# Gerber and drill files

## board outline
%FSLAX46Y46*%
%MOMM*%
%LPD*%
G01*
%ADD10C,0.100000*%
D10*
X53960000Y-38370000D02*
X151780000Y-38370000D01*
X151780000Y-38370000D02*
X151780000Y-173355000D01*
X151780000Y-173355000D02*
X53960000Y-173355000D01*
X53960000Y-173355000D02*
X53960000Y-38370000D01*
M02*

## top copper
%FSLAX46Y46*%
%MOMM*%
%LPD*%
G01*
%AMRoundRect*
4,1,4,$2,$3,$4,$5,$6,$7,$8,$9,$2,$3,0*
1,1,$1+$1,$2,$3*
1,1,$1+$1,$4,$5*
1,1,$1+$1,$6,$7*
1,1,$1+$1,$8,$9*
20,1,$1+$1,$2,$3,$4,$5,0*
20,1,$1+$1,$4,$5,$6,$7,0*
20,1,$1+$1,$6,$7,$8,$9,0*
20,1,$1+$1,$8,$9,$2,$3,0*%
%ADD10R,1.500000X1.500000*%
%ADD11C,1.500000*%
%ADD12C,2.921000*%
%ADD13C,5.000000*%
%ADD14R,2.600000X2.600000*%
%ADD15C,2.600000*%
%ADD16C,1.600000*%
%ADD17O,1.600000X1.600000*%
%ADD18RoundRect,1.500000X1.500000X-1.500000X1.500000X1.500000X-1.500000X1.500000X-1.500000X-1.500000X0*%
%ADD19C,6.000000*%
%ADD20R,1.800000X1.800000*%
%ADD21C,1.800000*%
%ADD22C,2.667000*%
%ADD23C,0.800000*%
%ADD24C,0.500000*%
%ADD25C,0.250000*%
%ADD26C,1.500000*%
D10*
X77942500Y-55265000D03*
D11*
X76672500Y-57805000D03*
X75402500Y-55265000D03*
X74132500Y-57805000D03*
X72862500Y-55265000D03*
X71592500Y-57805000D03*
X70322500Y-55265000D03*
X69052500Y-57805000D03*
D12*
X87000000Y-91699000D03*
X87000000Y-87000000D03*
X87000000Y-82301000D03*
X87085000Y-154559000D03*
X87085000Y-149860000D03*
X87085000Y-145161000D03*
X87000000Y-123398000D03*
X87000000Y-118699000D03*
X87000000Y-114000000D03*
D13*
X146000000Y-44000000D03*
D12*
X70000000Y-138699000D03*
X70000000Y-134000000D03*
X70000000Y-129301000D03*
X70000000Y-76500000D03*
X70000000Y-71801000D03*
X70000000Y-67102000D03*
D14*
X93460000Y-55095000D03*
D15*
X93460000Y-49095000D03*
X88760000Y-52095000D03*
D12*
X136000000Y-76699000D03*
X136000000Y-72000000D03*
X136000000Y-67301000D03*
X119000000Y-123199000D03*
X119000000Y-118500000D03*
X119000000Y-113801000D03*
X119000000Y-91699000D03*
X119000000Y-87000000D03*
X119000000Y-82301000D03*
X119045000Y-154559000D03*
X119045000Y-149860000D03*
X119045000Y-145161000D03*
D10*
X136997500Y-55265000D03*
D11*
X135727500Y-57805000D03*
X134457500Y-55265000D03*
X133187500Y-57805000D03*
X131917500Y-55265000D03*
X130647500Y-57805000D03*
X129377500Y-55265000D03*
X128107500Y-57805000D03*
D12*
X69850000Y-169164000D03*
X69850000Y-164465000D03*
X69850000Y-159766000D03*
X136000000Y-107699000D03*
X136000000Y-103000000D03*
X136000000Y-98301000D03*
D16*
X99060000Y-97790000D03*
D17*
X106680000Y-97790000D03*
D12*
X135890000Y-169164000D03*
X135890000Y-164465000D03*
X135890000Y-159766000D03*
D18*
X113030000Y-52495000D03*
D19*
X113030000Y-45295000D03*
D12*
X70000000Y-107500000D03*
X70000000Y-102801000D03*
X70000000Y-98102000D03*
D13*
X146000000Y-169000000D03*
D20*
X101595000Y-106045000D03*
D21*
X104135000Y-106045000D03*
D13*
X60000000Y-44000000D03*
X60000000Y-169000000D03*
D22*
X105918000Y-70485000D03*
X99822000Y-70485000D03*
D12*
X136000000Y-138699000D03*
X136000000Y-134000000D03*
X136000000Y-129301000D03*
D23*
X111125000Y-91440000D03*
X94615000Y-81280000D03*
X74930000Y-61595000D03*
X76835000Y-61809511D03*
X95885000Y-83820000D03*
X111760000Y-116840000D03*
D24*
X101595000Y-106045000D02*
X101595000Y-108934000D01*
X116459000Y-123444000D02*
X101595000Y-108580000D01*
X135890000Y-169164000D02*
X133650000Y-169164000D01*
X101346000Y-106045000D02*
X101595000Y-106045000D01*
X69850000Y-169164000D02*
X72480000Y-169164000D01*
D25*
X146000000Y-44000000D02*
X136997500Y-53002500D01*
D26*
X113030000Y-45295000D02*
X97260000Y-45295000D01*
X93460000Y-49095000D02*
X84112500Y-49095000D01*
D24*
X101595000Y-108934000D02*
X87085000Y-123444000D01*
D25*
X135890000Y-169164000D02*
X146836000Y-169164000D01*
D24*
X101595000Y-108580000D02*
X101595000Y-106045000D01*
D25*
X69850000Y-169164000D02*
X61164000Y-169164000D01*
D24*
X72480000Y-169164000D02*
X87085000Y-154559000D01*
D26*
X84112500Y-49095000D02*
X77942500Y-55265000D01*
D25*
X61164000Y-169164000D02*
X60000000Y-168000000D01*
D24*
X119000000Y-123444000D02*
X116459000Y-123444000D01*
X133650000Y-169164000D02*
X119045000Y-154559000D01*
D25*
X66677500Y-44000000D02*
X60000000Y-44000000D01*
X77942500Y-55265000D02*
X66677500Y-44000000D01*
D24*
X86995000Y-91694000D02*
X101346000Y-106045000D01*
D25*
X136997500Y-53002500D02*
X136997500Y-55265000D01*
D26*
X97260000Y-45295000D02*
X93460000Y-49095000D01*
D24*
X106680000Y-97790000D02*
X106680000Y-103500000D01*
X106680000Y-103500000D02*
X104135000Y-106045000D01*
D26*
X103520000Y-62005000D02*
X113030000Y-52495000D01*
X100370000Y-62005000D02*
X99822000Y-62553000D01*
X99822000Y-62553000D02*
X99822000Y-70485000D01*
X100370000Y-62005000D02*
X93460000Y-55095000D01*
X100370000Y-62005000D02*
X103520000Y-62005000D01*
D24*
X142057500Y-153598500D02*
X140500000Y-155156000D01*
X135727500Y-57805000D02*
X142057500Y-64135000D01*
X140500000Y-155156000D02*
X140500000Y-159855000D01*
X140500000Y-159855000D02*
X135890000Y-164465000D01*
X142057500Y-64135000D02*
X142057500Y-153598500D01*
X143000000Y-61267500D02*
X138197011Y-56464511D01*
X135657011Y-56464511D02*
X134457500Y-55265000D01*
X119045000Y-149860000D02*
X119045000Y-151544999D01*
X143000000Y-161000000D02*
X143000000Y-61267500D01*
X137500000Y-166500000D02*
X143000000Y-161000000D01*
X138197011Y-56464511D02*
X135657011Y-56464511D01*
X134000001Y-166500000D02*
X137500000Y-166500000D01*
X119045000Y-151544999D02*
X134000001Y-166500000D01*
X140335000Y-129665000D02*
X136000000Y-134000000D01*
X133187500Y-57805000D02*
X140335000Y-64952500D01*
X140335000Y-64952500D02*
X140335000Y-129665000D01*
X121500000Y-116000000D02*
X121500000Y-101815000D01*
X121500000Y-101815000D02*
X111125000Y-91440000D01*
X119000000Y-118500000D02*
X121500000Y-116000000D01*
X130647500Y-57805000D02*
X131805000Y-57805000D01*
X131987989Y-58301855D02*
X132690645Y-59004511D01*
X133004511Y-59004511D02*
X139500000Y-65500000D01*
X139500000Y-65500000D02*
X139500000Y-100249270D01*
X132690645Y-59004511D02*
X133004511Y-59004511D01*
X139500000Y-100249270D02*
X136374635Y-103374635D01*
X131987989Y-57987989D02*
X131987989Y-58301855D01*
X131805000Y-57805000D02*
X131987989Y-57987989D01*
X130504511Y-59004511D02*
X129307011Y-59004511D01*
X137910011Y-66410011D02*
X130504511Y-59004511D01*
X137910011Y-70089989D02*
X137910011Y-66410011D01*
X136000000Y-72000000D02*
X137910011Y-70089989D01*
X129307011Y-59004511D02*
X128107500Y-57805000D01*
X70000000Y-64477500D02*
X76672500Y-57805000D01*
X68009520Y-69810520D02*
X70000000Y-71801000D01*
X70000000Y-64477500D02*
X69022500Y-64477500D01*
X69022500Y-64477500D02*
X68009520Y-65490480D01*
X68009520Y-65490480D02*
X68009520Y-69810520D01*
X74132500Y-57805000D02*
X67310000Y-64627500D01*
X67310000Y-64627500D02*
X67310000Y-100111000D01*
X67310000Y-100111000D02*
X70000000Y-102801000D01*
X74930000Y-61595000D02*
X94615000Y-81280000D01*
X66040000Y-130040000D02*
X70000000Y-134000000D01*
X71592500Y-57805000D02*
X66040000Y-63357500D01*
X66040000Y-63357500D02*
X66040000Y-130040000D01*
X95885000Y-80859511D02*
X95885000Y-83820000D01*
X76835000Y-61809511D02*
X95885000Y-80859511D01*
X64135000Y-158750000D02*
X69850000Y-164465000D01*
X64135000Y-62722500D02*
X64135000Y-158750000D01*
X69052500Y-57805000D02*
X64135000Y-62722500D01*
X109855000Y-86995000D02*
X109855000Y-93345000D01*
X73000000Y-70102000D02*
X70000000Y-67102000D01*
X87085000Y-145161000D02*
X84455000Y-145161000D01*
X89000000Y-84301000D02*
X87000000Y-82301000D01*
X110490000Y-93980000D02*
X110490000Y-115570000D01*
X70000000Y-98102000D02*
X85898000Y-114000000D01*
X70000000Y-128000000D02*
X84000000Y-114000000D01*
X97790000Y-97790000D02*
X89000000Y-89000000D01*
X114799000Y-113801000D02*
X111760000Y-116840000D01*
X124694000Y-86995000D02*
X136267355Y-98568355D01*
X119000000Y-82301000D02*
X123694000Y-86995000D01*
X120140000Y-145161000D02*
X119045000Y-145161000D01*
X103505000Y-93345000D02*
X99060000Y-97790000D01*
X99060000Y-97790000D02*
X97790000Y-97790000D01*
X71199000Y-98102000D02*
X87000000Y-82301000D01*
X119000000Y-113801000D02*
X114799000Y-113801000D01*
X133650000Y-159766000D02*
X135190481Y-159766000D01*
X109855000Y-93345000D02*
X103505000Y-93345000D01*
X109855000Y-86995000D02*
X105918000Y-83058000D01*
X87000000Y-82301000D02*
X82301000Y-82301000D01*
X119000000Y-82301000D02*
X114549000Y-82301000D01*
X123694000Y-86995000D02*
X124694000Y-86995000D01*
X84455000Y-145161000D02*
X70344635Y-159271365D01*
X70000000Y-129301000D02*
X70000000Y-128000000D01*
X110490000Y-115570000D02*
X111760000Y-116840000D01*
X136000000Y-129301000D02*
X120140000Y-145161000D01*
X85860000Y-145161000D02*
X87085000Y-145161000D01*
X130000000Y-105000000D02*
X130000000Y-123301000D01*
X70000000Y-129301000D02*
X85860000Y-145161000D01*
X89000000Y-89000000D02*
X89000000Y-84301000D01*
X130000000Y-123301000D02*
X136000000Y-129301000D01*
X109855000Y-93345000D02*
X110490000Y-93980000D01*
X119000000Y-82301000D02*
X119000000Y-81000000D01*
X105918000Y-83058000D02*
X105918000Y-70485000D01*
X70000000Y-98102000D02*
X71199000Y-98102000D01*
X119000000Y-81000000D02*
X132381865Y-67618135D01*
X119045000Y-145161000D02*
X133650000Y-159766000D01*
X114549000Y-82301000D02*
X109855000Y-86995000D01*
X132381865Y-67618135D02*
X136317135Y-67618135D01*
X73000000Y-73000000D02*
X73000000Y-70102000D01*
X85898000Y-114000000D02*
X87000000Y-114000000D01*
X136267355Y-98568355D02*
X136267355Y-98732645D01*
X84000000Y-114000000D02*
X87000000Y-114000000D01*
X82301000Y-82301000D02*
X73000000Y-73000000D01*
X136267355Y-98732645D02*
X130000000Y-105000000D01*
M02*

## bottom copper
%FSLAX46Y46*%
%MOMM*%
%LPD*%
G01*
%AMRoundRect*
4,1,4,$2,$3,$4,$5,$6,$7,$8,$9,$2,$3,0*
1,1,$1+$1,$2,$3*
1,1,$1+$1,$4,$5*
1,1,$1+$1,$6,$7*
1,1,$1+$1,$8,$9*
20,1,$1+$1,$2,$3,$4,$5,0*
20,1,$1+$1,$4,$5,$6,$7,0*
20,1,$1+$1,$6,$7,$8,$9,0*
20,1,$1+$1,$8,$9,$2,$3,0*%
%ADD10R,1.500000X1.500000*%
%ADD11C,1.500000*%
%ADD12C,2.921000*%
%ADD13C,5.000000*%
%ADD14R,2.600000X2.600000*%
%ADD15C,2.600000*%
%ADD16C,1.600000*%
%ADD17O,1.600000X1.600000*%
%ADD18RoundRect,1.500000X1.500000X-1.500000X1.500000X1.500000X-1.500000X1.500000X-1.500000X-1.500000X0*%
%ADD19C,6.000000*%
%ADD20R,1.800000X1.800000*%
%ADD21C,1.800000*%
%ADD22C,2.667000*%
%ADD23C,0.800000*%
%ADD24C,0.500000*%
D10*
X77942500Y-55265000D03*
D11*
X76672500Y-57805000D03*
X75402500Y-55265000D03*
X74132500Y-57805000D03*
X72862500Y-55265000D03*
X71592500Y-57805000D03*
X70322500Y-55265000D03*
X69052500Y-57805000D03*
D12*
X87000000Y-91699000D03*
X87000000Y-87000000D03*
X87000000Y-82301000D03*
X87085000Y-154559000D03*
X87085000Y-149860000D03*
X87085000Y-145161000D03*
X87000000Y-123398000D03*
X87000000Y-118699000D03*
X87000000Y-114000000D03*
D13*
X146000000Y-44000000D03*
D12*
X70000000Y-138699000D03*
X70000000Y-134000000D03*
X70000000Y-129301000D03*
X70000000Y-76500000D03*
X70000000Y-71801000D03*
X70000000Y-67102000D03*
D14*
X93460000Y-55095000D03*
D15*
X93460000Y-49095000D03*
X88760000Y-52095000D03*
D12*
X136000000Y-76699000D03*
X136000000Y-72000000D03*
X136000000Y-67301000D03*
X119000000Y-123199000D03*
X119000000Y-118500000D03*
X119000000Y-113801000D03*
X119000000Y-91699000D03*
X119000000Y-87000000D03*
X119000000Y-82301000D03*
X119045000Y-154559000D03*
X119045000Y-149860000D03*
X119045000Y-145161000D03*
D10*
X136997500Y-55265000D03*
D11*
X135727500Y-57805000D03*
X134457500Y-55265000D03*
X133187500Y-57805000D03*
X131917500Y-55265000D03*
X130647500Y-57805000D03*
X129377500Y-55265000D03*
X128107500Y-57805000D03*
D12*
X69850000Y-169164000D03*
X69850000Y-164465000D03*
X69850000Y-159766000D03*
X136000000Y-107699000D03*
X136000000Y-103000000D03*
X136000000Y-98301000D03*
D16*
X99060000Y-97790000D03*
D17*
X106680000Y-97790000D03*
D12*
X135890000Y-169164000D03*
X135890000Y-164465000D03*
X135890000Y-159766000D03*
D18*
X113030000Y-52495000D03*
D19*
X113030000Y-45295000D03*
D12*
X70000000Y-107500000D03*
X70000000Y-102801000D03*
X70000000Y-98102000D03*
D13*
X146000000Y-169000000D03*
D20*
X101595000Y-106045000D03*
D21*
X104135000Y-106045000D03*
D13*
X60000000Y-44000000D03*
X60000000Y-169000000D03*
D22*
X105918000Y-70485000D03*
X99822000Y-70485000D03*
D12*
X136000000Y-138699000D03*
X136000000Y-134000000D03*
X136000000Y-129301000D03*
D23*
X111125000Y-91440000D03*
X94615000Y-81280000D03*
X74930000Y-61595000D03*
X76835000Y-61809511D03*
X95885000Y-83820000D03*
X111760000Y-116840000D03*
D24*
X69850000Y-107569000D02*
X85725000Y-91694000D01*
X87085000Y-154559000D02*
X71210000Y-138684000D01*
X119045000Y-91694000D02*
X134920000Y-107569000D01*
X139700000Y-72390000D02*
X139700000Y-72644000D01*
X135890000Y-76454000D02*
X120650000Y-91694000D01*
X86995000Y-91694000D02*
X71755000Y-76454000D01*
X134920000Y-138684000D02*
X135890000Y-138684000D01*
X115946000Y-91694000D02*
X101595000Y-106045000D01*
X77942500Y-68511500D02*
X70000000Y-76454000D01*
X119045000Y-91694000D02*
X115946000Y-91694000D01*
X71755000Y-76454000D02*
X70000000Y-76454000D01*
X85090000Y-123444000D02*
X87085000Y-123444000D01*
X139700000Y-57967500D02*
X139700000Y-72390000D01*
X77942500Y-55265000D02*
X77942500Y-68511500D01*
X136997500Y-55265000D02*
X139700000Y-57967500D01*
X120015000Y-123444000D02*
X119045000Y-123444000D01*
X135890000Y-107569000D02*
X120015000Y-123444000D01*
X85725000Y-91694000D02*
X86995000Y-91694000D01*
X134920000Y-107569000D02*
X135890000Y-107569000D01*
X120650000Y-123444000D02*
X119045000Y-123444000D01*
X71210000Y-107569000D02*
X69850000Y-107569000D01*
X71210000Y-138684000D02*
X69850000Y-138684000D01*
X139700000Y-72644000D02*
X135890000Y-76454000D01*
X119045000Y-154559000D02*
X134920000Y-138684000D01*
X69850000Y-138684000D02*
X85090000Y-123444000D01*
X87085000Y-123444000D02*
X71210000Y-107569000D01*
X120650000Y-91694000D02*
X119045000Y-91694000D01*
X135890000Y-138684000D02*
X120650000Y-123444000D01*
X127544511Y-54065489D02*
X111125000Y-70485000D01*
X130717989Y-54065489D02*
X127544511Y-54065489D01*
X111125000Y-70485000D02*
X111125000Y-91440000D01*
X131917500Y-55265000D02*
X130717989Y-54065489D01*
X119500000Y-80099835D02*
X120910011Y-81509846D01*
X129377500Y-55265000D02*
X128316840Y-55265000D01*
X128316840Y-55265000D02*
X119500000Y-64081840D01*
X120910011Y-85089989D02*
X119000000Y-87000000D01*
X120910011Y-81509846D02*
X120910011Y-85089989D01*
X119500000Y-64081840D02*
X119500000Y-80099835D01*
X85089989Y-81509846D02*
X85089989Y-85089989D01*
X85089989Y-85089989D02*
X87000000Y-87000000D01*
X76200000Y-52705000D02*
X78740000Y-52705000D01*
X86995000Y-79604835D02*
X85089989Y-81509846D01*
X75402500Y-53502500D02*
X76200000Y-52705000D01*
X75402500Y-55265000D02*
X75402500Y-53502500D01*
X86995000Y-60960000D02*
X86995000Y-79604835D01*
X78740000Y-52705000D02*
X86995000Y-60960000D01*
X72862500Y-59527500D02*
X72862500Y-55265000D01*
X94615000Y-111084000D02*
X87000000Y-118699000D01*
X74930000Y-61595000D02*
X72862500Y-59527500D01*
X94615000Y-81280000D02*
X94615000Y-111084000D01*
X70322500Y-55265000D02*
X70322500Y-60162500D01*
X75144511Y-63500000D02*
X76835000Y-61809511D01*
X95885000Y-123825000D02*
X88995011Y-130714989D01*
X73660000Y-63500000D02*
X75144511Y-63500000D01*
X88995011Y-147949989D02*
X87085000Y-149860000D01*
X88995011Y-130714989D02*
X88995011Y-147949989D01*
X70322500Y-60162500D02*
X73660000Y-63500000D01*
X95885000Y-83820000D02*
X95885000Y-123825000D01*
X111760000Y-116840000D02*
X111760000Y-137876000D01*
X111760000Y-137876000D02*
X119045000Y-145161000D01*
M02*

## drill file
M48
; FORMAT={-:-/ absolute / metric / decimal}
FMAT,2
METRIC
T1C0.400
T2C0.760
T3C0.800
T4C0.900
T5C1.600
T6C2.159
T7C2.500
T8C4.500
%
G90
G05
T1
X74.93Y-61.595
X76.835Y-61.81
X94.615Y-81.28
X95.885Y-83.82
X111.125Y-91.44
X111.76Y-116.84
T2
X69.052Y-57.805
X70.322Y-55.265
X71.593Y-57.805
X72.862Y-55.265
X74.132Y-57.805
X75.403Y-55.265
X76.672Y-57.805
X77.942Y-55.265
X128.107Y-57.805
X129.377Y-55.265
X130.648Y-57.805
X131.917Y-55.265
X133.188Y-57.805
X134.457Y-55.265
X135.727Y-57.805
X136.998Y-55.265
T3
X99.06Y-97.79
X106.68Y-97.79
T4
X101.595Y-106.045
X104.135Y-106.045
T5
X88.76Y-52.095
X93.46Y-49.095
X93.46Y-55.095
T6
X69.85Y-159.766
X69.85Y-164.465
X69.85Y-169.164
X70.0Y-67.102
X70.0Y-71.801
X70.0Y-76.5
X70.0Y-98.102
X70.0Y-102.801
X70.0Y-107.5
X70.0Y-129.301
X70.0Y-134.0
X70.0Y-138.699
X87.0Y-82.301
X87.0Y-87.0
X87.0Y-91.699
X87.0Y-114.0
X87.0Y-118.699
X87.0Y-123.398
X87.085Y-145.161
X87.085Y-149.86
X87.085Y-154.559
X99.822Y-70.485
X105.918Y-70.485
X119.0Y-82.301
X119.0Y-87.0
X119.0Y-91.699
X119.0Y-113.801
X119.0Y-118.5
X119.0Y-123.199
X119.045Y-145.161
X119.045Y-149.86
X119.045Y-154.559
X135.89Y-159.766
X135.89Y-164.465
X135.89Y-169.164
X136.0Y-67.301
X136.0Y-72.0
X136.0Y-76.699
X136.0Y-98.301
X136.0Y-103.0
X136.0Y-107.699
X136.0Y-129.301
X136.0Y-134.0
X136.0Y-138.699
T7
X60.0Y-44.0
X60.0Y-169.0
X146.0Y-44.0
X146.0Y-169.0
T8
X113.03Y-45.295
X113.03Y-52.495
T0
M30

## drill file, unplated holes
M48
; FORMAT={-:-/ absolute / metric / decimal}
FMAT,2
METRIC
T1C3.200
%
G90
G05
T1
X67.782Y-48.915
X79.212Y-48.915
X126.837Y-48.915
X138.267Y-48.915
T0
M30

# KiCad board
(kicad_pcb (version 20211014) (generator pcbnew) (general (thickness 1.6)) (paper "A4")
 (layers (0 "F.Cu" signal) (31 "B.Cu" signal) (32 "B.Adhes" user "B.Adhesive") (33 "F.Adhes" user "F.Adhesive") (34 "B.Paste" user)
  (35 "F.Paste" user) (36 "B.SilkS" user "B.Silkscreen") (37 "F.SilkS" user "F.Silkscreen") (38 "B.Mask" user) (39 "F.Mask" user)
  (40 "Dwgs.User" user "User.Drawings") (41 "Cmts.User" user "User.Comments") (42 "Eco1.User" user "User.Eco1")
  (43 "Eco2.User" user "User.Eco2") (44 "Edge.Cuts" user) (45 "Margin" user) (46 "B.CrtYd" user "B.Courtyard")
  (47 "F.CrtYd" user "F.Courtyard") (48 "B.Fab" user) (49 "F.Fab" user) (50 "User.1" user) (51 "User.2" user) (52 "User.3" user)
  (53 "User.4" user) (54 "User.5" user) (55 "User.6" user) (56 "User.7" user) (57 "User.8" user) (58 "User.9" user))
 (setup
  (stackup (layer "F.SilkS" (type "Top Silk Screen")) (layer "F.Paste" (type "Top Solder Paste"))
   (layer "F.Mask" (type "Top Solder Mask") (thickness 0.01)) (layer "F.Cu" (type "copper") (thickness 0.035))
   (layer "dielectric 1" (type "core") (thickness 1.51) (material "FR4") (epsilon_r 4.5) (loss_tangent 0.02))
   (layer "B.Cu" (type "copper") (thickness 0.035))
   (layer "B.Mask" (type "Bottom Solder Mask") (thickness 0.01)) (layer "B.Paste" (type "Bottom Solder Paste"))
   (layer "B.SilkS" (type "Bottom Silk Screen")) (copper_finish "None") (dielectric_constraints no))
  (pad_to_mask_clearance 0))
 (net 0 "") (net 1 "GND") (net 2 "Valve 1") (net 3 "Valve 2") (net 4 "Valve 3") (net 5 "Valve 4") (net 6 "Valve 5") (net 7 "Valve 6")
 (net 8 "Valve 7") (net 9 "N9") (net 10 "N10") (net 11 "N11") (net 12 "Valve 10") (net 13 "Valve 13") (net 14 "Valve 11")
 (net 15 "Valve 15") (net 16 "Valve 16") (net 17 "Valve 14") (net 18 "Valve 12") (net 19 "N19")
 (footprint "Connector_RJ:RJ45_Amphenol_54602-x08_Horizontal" (layer "F.Cu") (at 77.9425 55.265 180)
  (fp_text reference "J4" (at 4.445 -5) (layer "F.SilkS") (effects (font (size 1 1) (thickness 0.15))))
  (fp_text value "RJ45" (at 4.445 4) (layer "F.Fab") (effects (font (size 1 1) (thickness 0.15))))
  (pad "" np_thru_hole circle (at -1.27 6.35 180) (size 3.2 3.2) (drill 3.2) (layers *.Cu *.Mask))
  (pad "" np_thru_hole circle (at 10.16 6.35 180) (size 3.2 3.2) (drill 3.2) (layers *.Cu *.Mask))
  (pad "1" thru_hole rect (at 0 0 180) (size 1.5 1.5) (drill 0.76) (layers *.Cu *.Mask) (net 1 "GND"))
  (pad "2" thru_hole circle (at 1.27 -2.54 180) (size 1.5 1.5) (drill 0.76) (layers *.Cu *.Mask) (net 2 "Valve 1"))
  (pad "3" thru_hole circle (at 2.54 0 180) (size 1.5 1.5) (drill 0.76) (layers *.Cu *.Mask) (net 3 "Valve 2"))
  (pad "4" thru_hole circle (at 3.81 -2.54 180) (size 1.5 1.5) (drill 0.76) (layers *.Cu *.Mask) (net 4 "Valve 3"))
  (pad "5" thru_hole circle (at 5.08 0 180) (size 1.5 1.5) (drill 0.76) (layers *.Cu *.Mask) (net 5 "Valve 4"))
  (pad "6" thru_hole circle (at 6.35 -2.54 180) (size 1.5 1.5) (drill 0.76) (layers *.Cu *.Mask) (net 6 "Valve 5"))
  (pad "7" thru_hole circle (at 7.62 0 180) (size 1.5 1.5) (drill 0.76) (layers *.Cu *.Mask) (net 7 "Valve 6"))
  (pad "8" thru_hole circle (at 8.89 -2.54 180) (size 1.5 1.5) (drill 0.76) (layers *.Cu *.Mask) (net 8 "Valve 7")))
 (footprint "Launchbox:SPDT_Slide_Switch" (layer "F.Cu") (at 87 87 90)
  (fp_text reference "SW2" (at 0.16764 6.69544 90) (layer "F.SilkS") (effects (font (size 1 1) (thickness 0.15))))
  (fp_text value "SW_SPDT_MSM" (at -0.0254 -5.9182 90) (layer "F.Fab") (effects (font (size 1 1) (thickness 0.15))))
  (pad "1" thru_hole circle (at -4.699 0 90) (size 2.921 2.921) (drill 2.159) (layers *.Cu *.Mask) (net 1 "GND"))
  (pad "2" thru_hole circle (at 0 0 90) (size 2.921 2.921) (drill 2.159) (layers *.Cu *.Mask) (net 3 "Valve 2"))
  (pad "3" thru_hole circle (at 4.699 0 90) (size 2.921 2.921) (drill 2.159) (layers *.Cu *.Mask) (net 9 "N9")))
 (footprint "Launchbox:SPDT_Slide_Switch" (layer "F.Cu") (at 87.085 149.86 90)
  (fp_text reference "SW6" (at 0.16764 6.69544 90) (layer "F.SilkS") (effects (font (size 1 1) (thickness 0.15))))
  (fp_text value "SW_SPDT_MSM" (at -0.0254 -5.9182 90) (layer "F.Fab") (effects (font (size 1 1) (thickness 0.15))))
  (pad "1" thru_hole circle (at -4.699 0 90) (size 2.921 2.921) (drill 2.159) (layers *.Cu *.Mask) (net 1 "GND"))
  (pad "2" thru_hole circle (at 0 0 90) (size 2.921 2.921) (drill 2.159) (layers *.Cu *.Mask) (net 7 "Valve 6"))
  (pad "3" thru_hole circle (at 4.699 0 90) (size 2.921 2.921) (drill 2.159) (layers *.Cu *.Mask) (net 9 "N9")))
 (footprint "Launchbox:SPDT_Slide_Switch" (layer "F.Cu") (at 87 118.699 90)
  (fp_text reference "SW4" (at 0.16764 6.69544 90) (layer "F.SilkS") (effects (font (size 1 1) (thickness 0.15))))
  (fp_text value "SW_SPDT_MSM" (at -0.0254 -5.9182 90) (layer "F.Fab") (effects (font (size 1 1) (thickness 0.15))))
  (pad "1" thru_hole circle (at -4.699 0 90) (size 2.921 2.921) (drill 2.159) (layers *.Cu *.Mask) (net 1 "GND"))
  (pad "2" thru_hole circle (at 0 0 90) (size 2.921 2.921) (drill 2.159) (layers *.Cu *.Mask) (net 5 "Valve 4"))
  (pad "3" thru_hole circle (at 4.699 0 90) (size 2.921 2.921) (drill 2.159) (layers *.Cu *.Mask) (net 9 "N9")))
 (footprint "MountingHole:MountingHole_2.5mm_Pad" (layer "F.Cu") (at 146 44)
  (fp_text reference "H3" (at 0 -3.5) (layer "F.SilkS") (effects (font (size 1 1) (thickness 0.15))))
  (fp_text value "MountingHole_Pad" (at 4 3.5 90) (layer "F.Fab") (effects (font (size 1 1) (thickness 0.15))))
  (pad "1" thru_hole circle (at 0 0) (size 5 5) (drill 2.5) (layers *.Cu *.Mask) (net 1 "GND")))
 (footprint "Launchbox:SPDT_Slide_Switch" (layer "F.Cu") (at 70 134 90)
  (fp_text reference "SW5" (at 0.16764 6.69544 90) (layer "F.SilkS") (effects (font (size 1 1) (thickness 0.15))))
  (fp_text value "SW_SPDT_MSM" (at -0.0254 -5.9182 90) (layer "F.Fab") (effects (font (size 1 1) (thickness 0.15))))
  (pad "1" thru_hole circle (at -4.699 0 90) (size 2.921 2.921) (drill 2.159) (layers *.Cu *.Mask) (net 1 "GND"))
  (pad "2" thru_hole circle (at 0 0 90) (size 2.921 2.921) (drill 2.159) (layers *.Cu *.Mask) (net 6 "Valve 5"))
  (pad "3" thru_hole circle (at 4.699 0 90) (size 2.921 2.921) (drill 2.159) (layers *.Cu *.Mask) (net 9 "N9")))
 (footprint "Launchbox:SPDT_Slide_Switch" (layer "F.Cu") (at 70 71.801 90)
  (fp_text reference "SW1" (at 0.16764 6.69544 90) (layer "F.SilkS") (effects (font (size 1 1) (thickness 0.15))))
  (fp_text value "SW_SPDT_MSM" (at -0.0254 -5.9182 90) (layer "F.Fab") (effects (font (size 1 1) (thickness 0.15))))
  (pad "1" thru_hole circle (at -4.699 0 90) (size 2.921 2.921) (drill 2.159) (layers *.Cu *.Mask) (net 1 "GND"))
  (pad "2" thru_hole circle (at 0 0 90) (size 2.921 2.921) (drill 2.159) (layers *.Cu *.Mask) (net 2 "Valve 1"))
  (pad "3" thru_hole circle (at 4.699 0 90) (size 2.921 2.921) (drill 2.159) (layers *.Cu *.Mask) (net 9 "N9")))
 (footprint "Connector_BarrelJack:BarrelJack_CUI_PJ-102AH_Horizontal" (layer "F.Cu") (at 93.46 55.095 180)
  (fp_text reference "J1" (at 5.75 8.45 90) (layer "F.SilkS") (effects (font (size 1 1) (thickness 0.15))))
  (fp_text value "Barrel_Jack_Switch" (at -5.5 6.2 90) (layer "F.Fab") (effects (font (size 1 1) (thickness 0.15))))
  (pad "1" thru_hole rect (at 0 0 180) (size 2.6 2.6) (drill 1.6) (layers *.Cu *.Mask) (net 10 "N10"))
  (pad "2" thru_hole circle (at 0 6 180) (size 2.6 2.6) (drill 1.6) (layers *.Cu *.Mask) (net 1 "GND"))
  (pad "3" thru_hole circle (at 4.7 3 180) (size 2.6 2.6) (drill 1.6) (layers *.Cu *.Mask) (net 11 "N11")))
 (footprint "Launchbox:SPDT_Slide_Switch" (layer "F.Cu") (at 136 72 90)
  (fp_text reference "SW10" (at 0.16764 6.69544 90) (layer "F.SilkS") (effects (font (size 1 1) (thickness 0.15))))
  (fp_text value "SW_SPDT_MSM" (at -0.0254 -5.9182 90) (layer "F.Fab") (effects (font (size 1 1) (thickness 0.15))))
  (pad "1" thru_hole circle (at -4.699 0 90) (size 2.921 2.921) (drill 2.159) (layers *.Cu *.Mask) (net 1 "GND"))
  (pad "2" thru_hole circle (at 0 0 90) (size 2.921 2.921) (drill 2.159) (layers *.Cu *.Mask) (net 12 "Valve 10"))
  (pad "3" thru_hole circle (at 4.699 0 90) (size 2.921 2.921) (drill 2.159) (layers *.Cu *.Mask) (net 9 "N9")))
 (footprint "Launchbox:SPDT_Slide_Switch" (layer "F.Cu") (at 119 118.5 90)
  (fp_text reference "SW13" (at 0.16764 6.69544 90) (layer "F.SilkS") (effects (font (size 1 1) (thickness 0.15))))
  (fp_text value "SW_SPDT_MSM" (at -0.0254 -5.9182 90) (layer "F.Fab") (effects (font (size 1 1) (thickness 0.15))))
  (pad "1" thru_hole circle (at -4.699 0 90) (size 2.921 2.921) (drill 2.159) (layers *.Cu *.Mask) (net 1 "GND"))
  (pad "2" thru_hole circle (at 0 0 90) (size 2.921 2.921) (drill 2.159) (layers *.Cu *.Mask) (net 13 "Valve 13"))
  (pad "3" thru_hole circle (at 4.699 0 90) (size 2.921 2.921) (drill 2.159) (layers *.Cu *.Mask) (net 9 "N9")))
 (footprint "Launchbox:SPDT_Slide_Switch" (layer "F.Cu") (at 119 87 90)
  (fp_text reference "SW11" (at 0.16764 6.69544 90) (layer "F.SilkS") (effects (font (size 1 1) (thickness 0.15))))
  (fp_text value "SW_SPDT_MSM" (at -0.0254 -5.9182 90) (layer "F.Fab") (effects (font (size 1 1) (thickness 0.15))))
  (pad "1" thru_hole circle (at -4.699 0 90) (size 2.921 2.921) (drill 2.159) (layers *.Cu *.Mask) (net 1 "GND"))
  (pad "2" thru_hole circle (at 0 0 90) (size 2.921 2.921) (drill 2.159) (layers *.Cu *.Mask) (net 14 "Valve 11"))
  (pad "3" thru_hole circle (at 4.699 0 90) (size 2.921 2.921) (drill 2.159) (layers *.Cu *.Mask) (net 9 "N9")))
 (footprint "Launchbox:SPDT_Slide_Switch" (layer "F.Cu") (at 119.045 149.86 90)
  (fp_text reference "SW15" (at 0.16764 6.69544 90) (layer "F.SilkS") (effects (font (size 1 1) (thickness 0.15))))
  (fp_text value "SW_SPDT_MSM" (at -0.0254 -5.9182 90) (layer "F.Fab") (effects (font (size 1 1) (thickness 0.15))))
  (pad "1" thru_hole circle (at -4.699 0 90) (size 2.921 2.921) (drill 2.159) (layers *.Cu *.Mask) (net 1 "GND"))
  (pad "2" thru_hole circle (at 0 0 90) (size 2.921 2.921) (drill 2.159) (layers *.Cu *.Mask) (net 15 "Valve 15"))
  (pad "3" thru_hole circle (at 4.699 0 90) (size 2.921 2.921) (drill 2.159) (layers *.Cu *.Mask) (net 9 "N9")))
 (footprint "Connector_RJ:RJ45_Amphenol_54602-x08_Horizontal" (layer "F.Cu") (at 136.9975 55.265 180)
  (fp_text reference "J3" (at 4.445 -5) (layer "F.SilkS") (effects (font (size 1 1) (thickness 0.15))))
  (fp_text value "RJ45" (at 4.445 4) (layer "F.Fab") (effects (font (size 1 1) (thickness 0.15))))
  (pad "" np_thru_hole circle (at -1.27 6.35 180) (size 3.2 3.2) (drill 3.2) (layers *.Cu *.Mask))
  (pad "" np_thru_hole circle (at 10.16 6.35 180) (size 3.2 3.2) (drill 3.2) (layers *.Cu *.Mask))
  (pad "1" thru_hole rect (at 0 0 180) (size 1.5 1.5) (drill 0.76) (layers *.Cu *.Mask) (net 1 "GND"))
  (pad "2" thru_hole circle (at 1.27 -2.54 180) (size 1.5 1.5) (drill 0.76) (layers *.Cu *.Mask) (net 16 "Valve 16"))
  (pad "3" thru_hole circle (at 2.54 0 180) (size 1.5 1.5) (drill 0.76) (layers *.Cu *.Mask) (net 15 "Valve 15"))
  (pad "4" thru_hole circle (at 3.81 -2.54 180) (size 1.5 1.5) (drill 0.76) (layers *.Cu *.Mask) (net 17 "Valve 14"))
  (pad "5" thru_hole circle (at 5.08 0 180) (size 1.5 1.5) (drill 0.76) (layers *.Cu *.Mask) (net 13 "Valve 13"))
  (pad "6" thru_hole circle (at 6.35 -2.54 180) (size 1.5 1.5) (drill 0.76) (layers *.Cu *.Mask) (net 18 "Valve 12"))
  (pad "7" thru_hole circle (at 7.62 0 180) (size 1.5 1.5) (drill 0.76) (layers *.Cu *.Mask) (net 14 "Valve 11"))
  (pad "8" thru_hole circle (at 8.89 -2.54 180) (size 1.5 1.5) (drill 0.76) (layers *.Cu *.Mask) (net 12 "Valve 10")))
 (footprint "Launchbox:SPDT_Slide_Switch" (layer "F.Cu") (at 69.85 164.465 90)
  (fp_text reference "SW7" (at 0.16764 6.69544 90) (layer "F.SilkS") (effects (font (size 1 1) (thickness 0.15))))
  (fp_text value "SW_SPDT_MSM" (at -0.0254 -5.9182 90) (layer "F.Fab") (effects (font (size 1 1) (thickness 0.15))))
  (pad "1" thru_hole circle (at -4.699 0 90) (size 2.921 2.921) (drill 2.159) (layers *.Cu *.Mask) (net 1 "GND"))
  (pad "2" thru_hole circle (at 0 0 90) (size 2.921 2.921) (drill 2.159) (layers *.Cu *.Mask) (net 8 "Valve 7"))
  (pad "3" thru_hole circle (at 4.699 0 90) (size 2.921 2.921) (drill 2.159) (layers *.Cu *.Mask) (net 9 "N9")))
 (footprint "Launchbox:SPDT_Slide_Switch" (layer "F.Cu") (at 136 103 90)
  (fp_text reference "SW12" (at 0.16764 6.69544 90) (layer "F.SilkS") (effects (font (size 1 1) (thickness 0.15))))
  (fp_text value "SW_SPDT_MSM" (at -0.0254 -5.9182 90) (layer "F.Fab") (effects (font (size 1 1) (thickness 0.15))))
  (pad "1" thru_hole circle (at -4.699 0 90) (size 2.921 2.921) (drill 2.159) (layers *.Cu *.Mask) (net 1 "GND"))
  (pad "2" thru_hole circle (at 0 0 90) (size 2.921 2.921) (drill 2.159) (layers *.Cu *.Mask) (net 18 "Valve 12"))
  (pad "3" thru_hole circle (at 4.699 0 90) (size 2.921 2.921) (drill 2.159) (layers *.Cu *.Mask) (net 9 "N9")))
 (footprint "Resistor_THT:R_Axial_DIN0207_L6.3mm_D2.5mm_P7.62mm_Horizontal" (layer "F.Cu") (at 99.06 97.79)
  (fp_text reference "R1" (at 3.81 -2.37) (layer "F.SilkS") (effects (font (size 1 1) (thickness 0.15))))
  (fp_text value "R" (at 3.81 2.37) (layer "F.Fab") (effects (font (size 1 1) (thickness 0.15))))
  (pad "1" thru_hole circle (at 0 0) (size 1.6 1.6) (drill 0.8) (layers *.Cu *.Mask) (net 9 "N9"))
  (pad "2" thru_hole oval (at 7.62 0) (size 1.6 1.6) (drill 0.8) (layers *.Cu *.Mask) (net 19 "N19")))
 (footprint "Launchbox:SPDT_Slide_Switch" (layer "F.Cu") (at 135.89 164.465 90)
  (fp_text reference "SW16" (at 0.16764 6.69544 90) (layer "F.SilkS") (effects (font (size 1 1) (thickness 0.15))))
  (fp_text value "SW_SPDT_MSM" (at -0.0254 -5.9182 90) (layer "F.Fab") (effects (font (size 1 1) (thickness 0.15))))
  (pad "1" thru_hole circle (at -4.699 0 90) (size 2.921 2.921) (drill 2.159) (layers *.Cu *.Mask) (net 1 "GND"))
  (pad "2" thru_hole circle (at 0 0 90) (size 2.921 2.921) (drill 2.159) (layers *.Cu *.Mask) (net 16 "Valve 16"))
  (pad "3" thru_hole circle (at 4.699 0 90) (size 2.921 2.921) (drill 2.159) (layers *.Cu *.Mask) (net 9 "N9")))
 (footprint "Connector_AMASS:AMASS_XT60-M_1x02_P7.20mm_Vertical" (layer "F.Cu") (at 113.03 52.495 90)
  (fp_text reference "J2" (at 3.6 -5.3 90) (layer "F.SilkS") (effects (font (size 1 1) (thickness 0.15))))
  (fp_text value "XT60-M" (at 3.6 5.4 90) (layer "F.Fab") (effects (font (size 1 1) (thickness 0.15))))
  (pad "1" thru_hole roundrect (at 0 0 90) (size 6 6) (drill 4.5) (layers *.Cu *.Mask) (roundrect_rratio 0.25) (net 10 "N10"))
  (pad "2" thru_hole circle (at 7.2 0 90) (size 6 6) (drill 4.5) (layers *.Cu *.Mask) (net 1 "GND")))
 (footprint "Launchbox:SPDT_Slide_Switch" (layer "F.Cu") (at 70 102.801 90)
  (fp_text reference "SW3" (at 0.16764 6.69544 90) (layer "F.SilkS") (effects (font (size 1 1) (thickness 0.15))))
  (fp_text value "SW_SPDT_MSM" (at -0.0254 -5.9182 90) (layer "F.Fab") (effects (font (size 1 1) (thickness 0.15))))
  (pad "1" thru_hole circle (at -4.699 0 90) (size 2.921 2.921) (drill 2.159) (layers *.Cu *.Mask) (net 1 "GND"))
  (pad "2" thru_hole circle (at 0 0 90) (size 2.921 2.921) (drill 2.159) (layers *.Cu *.Mask) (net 4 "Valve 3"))
  (pad "3" thru_hole circle (at 4.699 0 90) (size 2.921 2.921) (drill 2.159) (layers *.Cu *.Mask) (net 9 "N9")))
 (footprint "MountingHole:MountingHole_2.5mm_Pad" (layer "F.Cu") (at 146 169)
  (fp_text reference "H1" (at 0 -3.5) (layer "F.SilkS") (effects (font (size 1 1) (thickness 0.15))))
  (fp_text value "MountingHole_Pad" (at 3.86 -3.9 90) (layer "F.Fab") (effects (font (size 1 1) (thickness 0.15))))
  (pad "1" thru_hole circle (at 0 0) (size 5 5) (drill 2.5) (layers *.Cu *.Mask) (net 1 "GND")))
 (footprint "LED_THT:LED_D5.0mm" (layer "F.Cu") (at 101.595 106.045)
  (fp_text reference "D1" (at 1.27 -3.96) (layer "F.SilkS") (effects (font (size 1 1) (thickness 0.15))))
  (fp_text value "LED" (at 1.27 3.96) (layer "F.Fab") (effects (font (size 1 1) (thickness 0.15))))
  (pad "1" thru_hole rect (at 0 0) (size 1.8 1.8) (drill 0.9) (layers *.Cu *.Mask) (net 1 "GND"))
  (pad "2" thru_hole circle (at 2.54 0) (size 1.8 1.8) (drill 0.9) (layers *.Cu *.Mask) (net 19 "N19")))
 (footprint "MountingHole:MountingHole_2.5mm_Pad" (layer "F.Cu") (at 60 44)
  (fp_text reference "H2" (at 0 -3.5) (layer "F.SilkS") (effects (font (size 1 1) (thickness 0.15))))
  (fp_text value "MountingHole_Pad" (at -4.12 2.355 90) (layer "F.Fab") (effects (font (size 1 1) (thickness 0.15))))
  (pad "1" thru_hole circle (at 0 0) (size 5 5) (drill 2.5) (layers *.Cu *.Mask) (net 1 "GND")))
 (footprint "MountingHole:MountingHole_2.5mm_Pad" (layer "F.Cu") (at 60 169)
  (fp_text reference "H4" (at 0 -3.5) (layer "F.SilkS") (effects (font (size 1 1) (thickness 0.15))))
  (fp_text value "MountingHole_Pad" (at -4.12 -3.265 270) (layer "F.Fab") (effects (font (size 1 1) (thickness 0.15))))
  (pad "1" thru_hole circle (at 0 0) (size 5 5) (drill 2.5) (layers *.Cu *.Mask) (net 1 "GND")))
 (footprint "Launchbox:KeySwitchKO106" (layer "F.Cu") (at 102.87 70.485 180)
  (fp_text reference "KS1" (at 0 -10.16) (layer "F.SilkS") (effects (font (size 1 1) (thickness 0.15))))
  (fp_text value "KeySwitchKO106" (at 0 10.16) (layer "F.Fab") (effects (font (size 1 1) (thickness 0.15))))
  (pad "1" thru_hole circle (at -3.048 0 180) (size 2.667 2.667) (drill 2.159) (layers *.Cu *.Mask) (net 9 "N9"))
  (pad "2" thru_hole circle (at 3.048 0 180) (size 2.667 2.667) (drill 2.159) (layers *.Cu *.Mask) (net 10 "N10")))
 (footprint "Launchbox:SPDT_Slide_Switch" (layer "F.Cu") (at 136 134 90)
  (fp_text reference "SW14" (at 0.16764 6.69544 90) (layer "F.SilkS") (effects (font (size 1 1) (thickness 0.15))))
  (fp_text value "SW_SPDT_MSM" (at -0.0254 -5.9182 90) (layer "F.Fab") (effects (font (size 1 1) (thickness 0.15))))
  (pad "1" thru_hole circle (at -4.699 0 90) (size 2.921 2.921) (drill 2.159) (layers *.Cu *.Mask) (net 1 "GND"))
  (pad "2" thru_hole circle (at 0 0 90) (size 2.921 2.921) (drill 2.159) (layers *.Cu *.Mask) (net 17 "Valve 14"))
  (pad "3" thru_hole circle (at 4.699 0 90) (size 2.921 2.921) (drill 2.159) (layers *.Cu *.Mask) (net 9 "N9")))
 (gr_rect (start 53.96 38.37) (end 151.78 173.355) (layer "Edge.Cuts") (width 0.1) (fill none))
 (segment (start 101.595 106.045) (end 101.595 108.934) (width 0.5) (layer "F.Cu") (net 1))
 (segment (start 116.459 123.444) (end 101.595 108.58) (width 0.5) (layer "F.Cu") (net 1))
 (segment (start 135.89 169.164) (end 133.65 169.164) (width 0.5) (layer "F.Cu") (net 1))
 (segment (start 101.346 106.045) (end 101.595 106.045) (width 0.5) (layer "F.Cu") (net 1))
 (segment (start 69.85 169.164) (end 72.48 169.164) (width 0.5) (layer "F.Cu") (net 1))
 (segment (start 146 44) (end 136.9975 53.0025) (width 0.25) (layer "F.Cu") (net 1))
 (segment (start 113.03 45.295) (end 97.26 45.295) (width 1.5) (layer "F.Cu") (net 1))
 (segment (start 93.46 49.095) (end 84.1125 49.095) (width 1.5) (layer "F.Cu") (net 1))
 (segment (start 101.595 108.934) (end 87.085 123.444) (width 0.5) (layer "F.Cu") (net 1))
 (segment (start 135.89 169.164) (end 146.836 169.164) (width 0.25) (layer "F.Cu") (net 1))
 (segment (start 101.595 108.58) (end 101.595 106.045) (width 0.5) (layer "F.Cu") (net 1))
 (segment (start 69.85 169.164) (end 61.164 169.164) (width 0.25) (layer "F.Cu") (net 1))
 (segment (start 72.48 169.164) (end 87.085 154.559) (width 0.5) (layer "F.Cu") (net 1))
 (segment (start 84.1125 49.095) (end 77.9425 55.265) (width 1.5) (layer "F.Cu") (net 1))
 (segment (start 61.164 169.164) (end 60 168) (width 0.25) (layer "F.Cu") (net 1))
 (segment (start 119 123.444) (end 116.459 123.444) (width 0.5) (layer "F.Cu") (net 1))
 (segment (start 133.65 169.164) (end 119.045 154.559) (width 0.5) (layer "F.Cu") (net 1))
 (segment (start 66.6775 44) (end 60 44) (width 0.25) (layer "F.Cu") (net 1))
 (segment (start 77.9425 55.265) (end 66.6775 44) (width 0.25) (layer "F.Cu") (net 1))
 (segment (start 86.995 91.694) (end 101.346 106.045) (width 0.5) (layer "F.Cu") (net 1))
 (segment (start 136.9975 53.0025) (end 136.9975 55.265) (width 0.25) (layer "F.Cu") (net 1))
 (segment (start 97.26 45.295) (end 93.46 49.095) (width 1.5) (layer "F.Cu") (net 1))
 (segment (start 69.85 107.569) (end 85.725 91.694) (width 0.5) (layer "B.Cu") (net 1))
 (segment (start 87.085 154.559) (end 71.21 138.684) (width 0.5) (layer "B.Cu") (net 1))
 (segment (start 119.045 91.694) (end 134.92 107.569) (width 0.5) (layer "B.Cu") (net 1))
 (segment (start 139.7 72.39) (end 139.7 72.644) (width 0.5) (layer "B.Cu") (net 1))
 (segment (start 135.89 76.454) (end 120.65 91.694) (width 0.5) (layer "B.Cu") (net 1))
 (segment (start 86.995 91.694) (end 71.755 76.454) (width 0.5) (layer "B.Cu") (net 1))
 (segment (start 134.92 138.684) (end 135.89 138.684) (width 0.5) (layer "B.Cu") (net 1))
 (segment (start 115.946 91.694) (end 101.595 106.045) (width 0.5) (layer "B.Cu") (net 1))
 (segment (start 77.9425 68.5115) (end 70 76.454) (width 0.5) (layer "B.Cu") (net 1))
 (segment (start 119.045 91.694) (end 115.946 91.694) (width 0.5) (layer "B.Cu") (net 1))
 (segment (start 71.755 76.454) (end 70 76.454) (width 0.5) (layer "B.Cu") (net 1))
 (segment (start 85.09 123.444) (end 87.085 123.444) (width 0.5) (layer "B.Cu") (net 1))
 (segment (start 139.7 57.9675) (end 139.7 72.39) (width 0.5) (layer "B.Cu") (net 1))
 (segment (start 77.9425 55.265) (end 77.9425 68.5115) (width 0.5) (layer "B.Cu") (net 1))
 (segment (start 136.9975 55.265) (end 139.7 57.9675) (width 0.5) (layer "B.Cu") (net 1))
 (segment (start 120.015 123.444) (end 119.045 123.444) (width 0.5) (layer "B.Cu") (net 1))
 (segment (start 135.89 107.569) (end 120.015 123.444) (width 0.5) (layer "B.Cu") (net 1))
 (segment (start 85.725 91.694) (end 86.995 91.694) (width 0.5) (layer "B.Cu") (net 1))
 (segment (start 134.92 107.569) (end 135.89 107.569) (width 0.5) (layer "B.Cu") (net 1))
 (segment (start 120.65 123.444) (end 119.045 123.444) (width 0.5) (layer "B.Cu") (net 1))
 (segment (start 71.21 107.569) (end 69.85 107.569) (width 0.5) (layer "B.Cu") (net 1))
 (segment (start 71.21 138.684) (end 69.85 138.684) (width 0.5) (layer "B.Cu") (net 1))
 (segment (start 139.7 72.644) (end 135.89 76.454) (width 0.5) (layer "B.Cu") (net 1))
 (segment (start 119.045 154.559) (end 134.92 138.684) (width 0.5) (layer "B.Cu") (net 1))
 (segment (start 69.85 138.684) (end 85.09 123.444) (width 0.5) (layer "B.Cu") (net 1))
 (segment (start 87.085 123.444) (end 71.21 107.569) (width 0.5) (layer "B.Cu") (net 1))
 (segment (start 120.65 91.694) (end 119.045 91.694) (width 0.5) (layer "B.Cu") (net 1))
 (segment (start 135.89 138.684) (end 120.65 123.444) (width 0.5) (layer "B.Cu") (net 1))
 (segment (start 106.68 97.79) (end 106.68 103.5) (width 0.5) (layer "F.Cu") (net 19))
 (segment (start 106.68 103.5) (end 104.135 106.045) (width 0.5) (layer "F.Cu") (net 19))
 (segment (start 103.52 62.005) (end 113.03 52.495) (width 1.5) (layer "F.Cu") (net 10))
 (segment (start 100.37 62.005) (end 99.822 62.553) (width 1.5) (layer "F.Cu") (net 10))
 (segment (start 99.822 62.553) (end 99.822 70.485) (width 1.5) (layer "F.Cu") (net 10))
 (segment (start 100.37 62.005) (end 93.46 55.095) (width 1.5) (layer "F.Cu") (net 10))
 (segment (start 100.37 62.005) (end 103.52 62.005) (width 1.5) (layer "F.Cu") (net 10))
 (segment (start 142.0575 153.5985) (end 140.5 155.156) (width 0.5) (layer "F.Cu") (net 16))
 (segment (start 135.7275 57.805) (end 142.0575 64.135) (width 0.5) (layer "F.Cu") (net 16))
 (segment (start 140.5 155.156) (end 140.5 159.855) (width 0.5) (layer "F.Cu") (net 16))
 (segment (start 140.5 159.855) (end 135.89 164.465) (width 0.5) (layer "F.Cu") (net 16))
 (segment (start 142.0575 64.135) (end 142.0575 153.5985) (width 0.5) (layer "F.Cu") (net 16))
 (segment (start 143 61.2675) (end 138.197011 56.464511) (width 0.5) (layer "F.Cu") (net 15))
 (segment (start 135.657011 56.464511) (end 134.4575 55.265) (width 0.5) (layer "F.Cu") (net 15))
 (segment (start 119.045 149.86) (end 119.045 151.544999) (width 0.5) (layer "F.Cu") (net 15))
 (segment (start 143 161) (end 143 61.2675) (width 0.5) (layer "F.Cu") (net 15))
 (segment (start 137.5 166.5) (end 143 161) (width 0.5) (layer "F.Cu") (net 15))
 (segment (start 138.197011 56.464511) (end 135.657011 56.464511) (width 0.5) (layer "F.Cu") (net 15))
 (segment (start 134.000001 166.5) (end 137.5 166.5) (width 0.5) (layer "F.Cu") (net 15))
 (segment (start 119.045 151.544999) (end 134.000001 166.5) (width 0.5) (layer "F.Cu") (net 15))
 (segment (start 140.335 129.665) (end 136 134) (width 0.5) (layer "F.Cu") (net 17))
 (segment (start 133.1875 57.805) (end 140.335 64.9525) (width 0.5) (layer "F.Cu") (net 17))
 (segment (start 140.335 64.9525) (end 140.335 129.665) (width 0.5) (layer "F.Cu") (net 17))
 (segment (start 121.5 116) (end 121.5 101.815) (width 0.5) (layer "F.Cu") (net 13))
 (segment (start 121.5 101.815) (end 111.125 91.44) (width 0.5) (layer "F.Cu") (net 13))
 (segment (start 119 118.5) (end 121.5 116) (width 0.5) (layer "F.Cu") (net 13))
 (via (at 111.125 91.44) (size 0.8) (drill 0.4) (layers "F.Cu" "B.Cu") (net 13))
 (segment (start 127.544511 54.065489) (end 111.125 70.485) (width 0.5) (layer "B.Cu") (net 13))
 (segment (start 130.717989 54.065489) (end 127.544511 54.065489) (width 0.5) (layer "B.Cu") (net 13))
 (segment (start 111.125 70.485) (end 111.125 91.44) (width 0.5) (layer "B.Cu") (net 13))
 (segment (start 131.9175 55.265) (end 130.717989 54.065489) (width 0.5) (layer "B.Cu") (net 13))
 (segment (start 130.6475 57.805) (end 131.805 57.805) (width 0.5) (layer "F.Cu") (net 18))
 (segment (start 131.987989 58.301855) (end 132.690645 59.004511) (width 0.5) (layer "F.Cu") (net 18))
 (segment (start 133.004511 59.004511) (end 139.5 65.5) (width 0.5) (layer "F.Cu") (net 18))
 (segment (start 139.5 65.5) (end 139.5 100.24927) (width 0.5) (layer "F.Cu") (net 18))
 (segment (start 132.690645 59.004511) (end 133.004511 59.004511) (width 0.5) (layer "F.Cu") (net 18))
 (segment (start 139.5 100.24927) (end 136.374635 103.374635) (width 0.5) (layer "F.Cu") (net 18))
 (segment (start 131.987989 57.987989) (end 131.987989 58.301855) (width 0.5) (layer "F.Cu") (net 18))
 (segment (start 131.805 57.805) (end 131.987989 57.987989) (width 0.5) (layer "F.Cu") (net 18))
 (segment (start 119.5 80.099835) (end 120.910011 81.509846) (width 0.5) (layer "B.Cu") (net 14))
 (segment (start 129.3775 55.265) (end 128.31684 55.265) (width 0.5) (layer "B.Cu") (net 14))
 (segment (start 128.31684 55.265) (end 119.5 64.08184) (width 0.5) (layer "B.Cu") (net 14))
 (segment (start 120.910011 85.089989) (end 119 87) (width 0.5) (layer "B.Cu") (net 14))
 (segment (start 120.910011 81.509846) (end 120.910011 85.089989) (width 0.5) (layer "B.Cu") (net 14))
 (segment (start 119.5 64.08184) (end 119.5 80.099835) (width 0.5) (layer "B.Cu") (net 14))
 (segment (start 130.504511 59.004511) (end 129.307011 59.004511) (width 0.5) (layer "F.Cu") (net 12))
 (segment (start 137.910011 66.410011) (end 130.504511 59.004511) (width 0.5) (layer "F.Cu") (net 12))
 (segment (start 137.910011 70.089989) (end 137.910011 66.410011) (width 0.5) (layer "F.Cu") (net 12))
 (segment (start 136 72) (end 137.910011 70.089989) (width 0.5) (layer "F.Cu") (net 12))
 (segment (start 129.307011 59.004511) (end 128.1075 57.805) (width 0.5) (layer "F.Cu") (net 12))
 (segment (start 70 64.4775) (end 76.6725 57.805) (width 0.5) (layer "F.Cu") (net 2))
 (segment (start 68.00952 69.81052) (end 70 71.801) (width 0.5) (layer "F.Cu") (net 2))
 (segment (start 70 64.4775) (end 69.0225 64.4775) (width 0.5) (layer "F.Cu") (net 2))
 (segment (start 69.0225 64.4775) (end 68.00952 65.49048) (width 0.5) (layer "F.Cu") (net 2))
 (segment (start 68.00952 65.49048) (end 68.00952 69.81052) (width 0.5) (layer "F.Cu") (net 2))
 (segment (start 85.089989 81.509846) (end 85.089989 85.089989) (width 0.5) (layer "B.Cu") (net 3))
 (segment (start 85.089989 85.089989) (end 87 87) (width 0.5) (layer "B.Cu") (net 3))
 (segment (start 76.2 52.705) (end 78.74 52.705) (width 0.5) (layer "B.Cu") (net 3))
 (segment (start 86.995 79.604835) (end 85.089989 81.509846) (width 0.5) (layer "B.Cu") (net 3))
 (segment (start 75.4025 53.5025) (end 76.2 52.705) (width 0.5) (layer "B.Cu") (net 3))
 (segment (start 75.4025 55.265) (end 75.4025 53.5025) (width 0.5) (layer "B.Cu") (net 3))
 (segment (start 86.995 60.96) (end 86.995 79.604835) (width 0.5) (layer "B.Cu") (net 3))
 (segment (start 78.74 52.705) (end 86.995 60.96) (width 0.5) (layer "B.Cu") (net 3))
 (segment (start 74.1325 57.805) (end 67.31 64.6275) (width 0.5) (layer "F.Cu") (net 4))
 (segment (start 67.31 64.6275) (end 67.31 100.111) (width 0.5) (layer "F.Cu") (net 4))
 (segment (start 67.31 100.111) (end 70 102.801) (width 0.5) (layer "F.Cu") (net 4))
 (segment (start 74.93 61.595) (end 94.615 81.28) (width 0.5) (layer "F.Cu") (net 5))
 (via (at 94.615 81.28) (size 0.8) (drill 0.4) (layers "F.Cu" "B.Cu") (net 5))
 (via (at 74.93 61.595) (size 0.8) (drill 0.4) (layers "F.Cu" "B.Cu") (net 5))
 (segment (start 72.8625 59.5275) (end 72.8625 55.265) (width 0.5) (layer "B.Cu") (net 5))
 (segment (start 94.615 111.084) (end 87 118.699) (width 0.5) (layer "B.Cu") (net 5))
 (segment (start 74.93 61.595) (end 72.8625 59.5275) (width 0.5) (layer "B.Cu") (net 5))
 (segment (start 94.615 81.28) (end 94.615 111.084) (width 0.5) (layer "B.Cu") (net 5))
 (segment (start 66.04 130.04) (end 70 134) (width 0.5) (layer "F.Cu") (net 6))
 (segment (start 71.5925 57.805) (end 66.04 63.3575) (width 0.5) (layer "F.Cu") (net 6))
 (segment (start 66.04 63.3575) (end 66.04 130.04) (width 0.5) (layer "F.Cu") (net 6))
 (segment (start 95.885 80.859511) (end 95.885 83.82) (width 0.5) (layer "F.Cu") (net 7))
 (segment (start 76.835 61.809511) (end 95.885 80.859511) (width 0.5) (layer "F.Cu") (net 7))
 (via (at 76.835 61.809511) (size 0.8) (drill 0.4) (layers "F.Cu" "B.Cu") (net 7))
 (via (at 95.885 83.82) (size 0.8) (drill 0.4) (layers "F.Cu" "B.Cu") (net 7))
 (segment (start 70.3225 55.265) (end 70.3225 60.1625) (width 0.5) (layer "B.Cu") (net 7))
 (segment (start 75.144511 63.5) (end 76.835 61.809511) (width 0.5) (layer "B.Cu") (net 7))
 (segment (start 95.885 123.825) (end 88.995011 130.714989) (width 0.5) (layer "B.Cu") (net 7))
 (segment (start 73.66 63.5) (end 75.144511 63.5) (width 0.5) (layer "B.Cu") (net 7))
 (segment (start 88.995011 147.949989) (end 87.085 149.86) (width 0.5) (layer "B.Cu") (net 7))
 (segment (start 88.995011 130.714989) (end 88.995011 147.949989) (width 0.5) (layer "B.Cu") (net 7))
 (segment (start 70.3225 60.1625) (end 73.66 63.5) (width 0.5) (layer "B.Cu") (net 7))
 (segment (start 95.885 83.82) (end 95.885 123.825) (width 0.5) (layer "B.Cu") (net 7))
 (segment (start 64.135 158.75) (end 69.85 164.465) (width 0.5) (layer "F.Cu") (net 8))
 (segment (start 64.135 62.7225) (end 64.135 158.75) (width 0.5) (layer "F.Cu") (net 8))
 (segment (start 69.0525 57.805) (end 64.135 62.7225) (width 0.5) (layer "F.Cu") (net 8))
 (segment (start 109.855 86.995) (end 109.855 93.345) (width 0.5) (layer "F.Cu") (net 9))
 (segment (start 73 70.102) (end 70 67.102) (width 0.5) (layer "F.Cu") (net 9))
 (segment (start 87.085 145.161) (end 84.455 145.161) (width 0.5) (layer "F.Cu") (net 9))
 (segment (start 89 84.301) (end 87 82.301) (width 0.5) (layer "F.Cu") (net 9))
 (segment (start 110.49 93.98) (end 110.49 115.57) (width 0.5) (layer "F.Cu") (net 9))
 (segment (start 70 98.102) (end 85.898 114) (width 0.5) (layer "F.Cu") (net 9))
 (segment (start 70 128) (end 84 114) (width 0.5) (layer "F.Cu") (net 9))
 (segment (start 97.79 97.79) (end 89 89) (width 0.5) (layer "F.Cu") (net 9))
 (segment (start 114.799 113.801) (end 111.76 116.84) (width 0.5) (layer "F.Cu") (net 9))
 (segment (start 124.694 86.995) (end 136.267355 98.568355) (width 0.5) (layer "F.Cu") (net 9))
 (segment (start 119 82.301) (end 123.694 86.995) (width 0.5) (layer "F.Cu") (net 9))
 (segment (start 120.14 145.161) (end 119.045 145.161) (width 0.5) (layer "F.Cu") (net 9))
 (segment (start 103.505 93.345) (end 99.06 97.79) (width 0.5) (layer "F.Cu") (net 9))
 (segment (start 99.06 97.79) (end 97.79 97.79) (width 0.5) (layer "F.Cu") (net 9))
 (segment (start 71.199 98.102) (end 87 82.301) (width 0.5) (layer "F.Cu") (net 9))
 (segment (start 119 113.801) (end 114.799 113.801) (width 0.5) (layer "F.Cu") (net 9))
 (segment (start 133.65 159.766) (end 135.190481 159.766) (width 0.5) (layer "F.Cu") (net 9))
 (segment (start 109.855 93.345) (end 103.505 93.345) (width 0.5) (layer "F.Cu") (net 9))
 (segment (start 109.855 86.995) (end 105.918 83.058) (width 0.5) (layer "F.Cu") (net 9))
 (segment (start 87 82.301) (end 82.301 82.301) (width 0.5) (layer "F.Cu") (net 9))
 (segment (start 119 82.301) (end 114.549 82.301) (width 0.5) (layer "F.Cu") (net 9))
 (segment (start 123.694 86.995) (end 124.694 86.995) (width 0.5) (layer "F.Cu") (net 9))
 (segment (start 84.455 145.161) (end 70.344635 159.271365) (width 0.5) (layer "F.Cu") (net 9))
 (segment (start 70 129.301) (end 70 128) (width 0.5) (layer "F.Cu") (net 9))
 (segment (start 110.49 115.57) (end 111.76 116.84) (width 0.5) (layer "F.Cu") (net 9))
 (segment (start 136 129.301) (end 120.14 145.161) (width 0.5) (layer "F.Cu") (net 9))
 (segment (start 85.86 145.161) (end 87.085 145.161) (width 0.5) (layer "F.Cu") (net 9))
 (segment (start 130 105) (end 130 123.301) (width 0.5) (layer "F.Cu") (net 9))
 (segment (start 70 129.301) (end 85.86 145.161) (width 0.5) (layer "F.Cu") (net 9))
 (segment (start 89 89) (end 89 84.301) (width 0.5) (layer "F.Cu") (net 9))
 (segment (start 130 123.301) (end 136 129.301) (width 0.5) (layer "F.Cu") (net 9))
 (segment (start 109.855 93.345) (end 110.49 93.98) (width 0.5) (layer "F.Cu") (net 9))
 (segment (start 119 82.301) (end 119 81) (width 0.5) (layer "F.Cu") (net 9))
 (segment (start 105.918 83.058) (end 105.918 70.485) (width 0.5) (layer "F.Cu") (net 9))
 (segment (start 70 98.102) (end 71.199 98.102) (width 0.5) (layer "F.Cu") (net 9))
 (segment (start 119 81) (end 132.381865 67.618135) (width 0.5) (layer "F.Cu") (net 9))
 (segment (start 119.045 145.161) (end 133.65 159.766) (width 0.5) (layer "F.Cu") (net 9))
 (segment (start 114.549 82.301) (end 109.855 86.995) (width 0.5) (layer "F.Cu") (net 9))
 (segment (start 132.381865 67.618135) (end 136.317135 67.618135) (width 0.5) (layer "F.Cu") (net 9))
 (segment (start 73 73) (end 73 70.102) (width 0.5) (layer "F.Cu") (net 9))
 (segment (start 85.898 114) (end 87 114) (width 0.5) (layer "F.Cu") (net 9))
 (segment (start 136.267355 98.568355) (end 136.267355 98.732645) (width 0.5) (layer "F.Cu") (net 9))
 (segment (start 84 114) (end 87 114) (width 0.5) (layer "F.Cu") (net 9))
 (segment (start 82.301 82.301) (end 73 73) (width 0.5) (layer "F.Cu") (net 9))
 (segment (start 136.267355 98.732645) (end 130 105) (width 0.5) (layer "F.Cu") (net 9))
 (via (at 111.76 116.84) (size 0.8) (drill 0.4) (layers "F.Cu" "B.Cu") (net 9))
 (segment (start 111.76 116.84) (end 111.76 137.876) (width 0.5) (layer "B.Cu") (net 9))
 (segment (start 111.76 137.876) (end 119.045 145.161) (width 0.5) (layer "B.Cu") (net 9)))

